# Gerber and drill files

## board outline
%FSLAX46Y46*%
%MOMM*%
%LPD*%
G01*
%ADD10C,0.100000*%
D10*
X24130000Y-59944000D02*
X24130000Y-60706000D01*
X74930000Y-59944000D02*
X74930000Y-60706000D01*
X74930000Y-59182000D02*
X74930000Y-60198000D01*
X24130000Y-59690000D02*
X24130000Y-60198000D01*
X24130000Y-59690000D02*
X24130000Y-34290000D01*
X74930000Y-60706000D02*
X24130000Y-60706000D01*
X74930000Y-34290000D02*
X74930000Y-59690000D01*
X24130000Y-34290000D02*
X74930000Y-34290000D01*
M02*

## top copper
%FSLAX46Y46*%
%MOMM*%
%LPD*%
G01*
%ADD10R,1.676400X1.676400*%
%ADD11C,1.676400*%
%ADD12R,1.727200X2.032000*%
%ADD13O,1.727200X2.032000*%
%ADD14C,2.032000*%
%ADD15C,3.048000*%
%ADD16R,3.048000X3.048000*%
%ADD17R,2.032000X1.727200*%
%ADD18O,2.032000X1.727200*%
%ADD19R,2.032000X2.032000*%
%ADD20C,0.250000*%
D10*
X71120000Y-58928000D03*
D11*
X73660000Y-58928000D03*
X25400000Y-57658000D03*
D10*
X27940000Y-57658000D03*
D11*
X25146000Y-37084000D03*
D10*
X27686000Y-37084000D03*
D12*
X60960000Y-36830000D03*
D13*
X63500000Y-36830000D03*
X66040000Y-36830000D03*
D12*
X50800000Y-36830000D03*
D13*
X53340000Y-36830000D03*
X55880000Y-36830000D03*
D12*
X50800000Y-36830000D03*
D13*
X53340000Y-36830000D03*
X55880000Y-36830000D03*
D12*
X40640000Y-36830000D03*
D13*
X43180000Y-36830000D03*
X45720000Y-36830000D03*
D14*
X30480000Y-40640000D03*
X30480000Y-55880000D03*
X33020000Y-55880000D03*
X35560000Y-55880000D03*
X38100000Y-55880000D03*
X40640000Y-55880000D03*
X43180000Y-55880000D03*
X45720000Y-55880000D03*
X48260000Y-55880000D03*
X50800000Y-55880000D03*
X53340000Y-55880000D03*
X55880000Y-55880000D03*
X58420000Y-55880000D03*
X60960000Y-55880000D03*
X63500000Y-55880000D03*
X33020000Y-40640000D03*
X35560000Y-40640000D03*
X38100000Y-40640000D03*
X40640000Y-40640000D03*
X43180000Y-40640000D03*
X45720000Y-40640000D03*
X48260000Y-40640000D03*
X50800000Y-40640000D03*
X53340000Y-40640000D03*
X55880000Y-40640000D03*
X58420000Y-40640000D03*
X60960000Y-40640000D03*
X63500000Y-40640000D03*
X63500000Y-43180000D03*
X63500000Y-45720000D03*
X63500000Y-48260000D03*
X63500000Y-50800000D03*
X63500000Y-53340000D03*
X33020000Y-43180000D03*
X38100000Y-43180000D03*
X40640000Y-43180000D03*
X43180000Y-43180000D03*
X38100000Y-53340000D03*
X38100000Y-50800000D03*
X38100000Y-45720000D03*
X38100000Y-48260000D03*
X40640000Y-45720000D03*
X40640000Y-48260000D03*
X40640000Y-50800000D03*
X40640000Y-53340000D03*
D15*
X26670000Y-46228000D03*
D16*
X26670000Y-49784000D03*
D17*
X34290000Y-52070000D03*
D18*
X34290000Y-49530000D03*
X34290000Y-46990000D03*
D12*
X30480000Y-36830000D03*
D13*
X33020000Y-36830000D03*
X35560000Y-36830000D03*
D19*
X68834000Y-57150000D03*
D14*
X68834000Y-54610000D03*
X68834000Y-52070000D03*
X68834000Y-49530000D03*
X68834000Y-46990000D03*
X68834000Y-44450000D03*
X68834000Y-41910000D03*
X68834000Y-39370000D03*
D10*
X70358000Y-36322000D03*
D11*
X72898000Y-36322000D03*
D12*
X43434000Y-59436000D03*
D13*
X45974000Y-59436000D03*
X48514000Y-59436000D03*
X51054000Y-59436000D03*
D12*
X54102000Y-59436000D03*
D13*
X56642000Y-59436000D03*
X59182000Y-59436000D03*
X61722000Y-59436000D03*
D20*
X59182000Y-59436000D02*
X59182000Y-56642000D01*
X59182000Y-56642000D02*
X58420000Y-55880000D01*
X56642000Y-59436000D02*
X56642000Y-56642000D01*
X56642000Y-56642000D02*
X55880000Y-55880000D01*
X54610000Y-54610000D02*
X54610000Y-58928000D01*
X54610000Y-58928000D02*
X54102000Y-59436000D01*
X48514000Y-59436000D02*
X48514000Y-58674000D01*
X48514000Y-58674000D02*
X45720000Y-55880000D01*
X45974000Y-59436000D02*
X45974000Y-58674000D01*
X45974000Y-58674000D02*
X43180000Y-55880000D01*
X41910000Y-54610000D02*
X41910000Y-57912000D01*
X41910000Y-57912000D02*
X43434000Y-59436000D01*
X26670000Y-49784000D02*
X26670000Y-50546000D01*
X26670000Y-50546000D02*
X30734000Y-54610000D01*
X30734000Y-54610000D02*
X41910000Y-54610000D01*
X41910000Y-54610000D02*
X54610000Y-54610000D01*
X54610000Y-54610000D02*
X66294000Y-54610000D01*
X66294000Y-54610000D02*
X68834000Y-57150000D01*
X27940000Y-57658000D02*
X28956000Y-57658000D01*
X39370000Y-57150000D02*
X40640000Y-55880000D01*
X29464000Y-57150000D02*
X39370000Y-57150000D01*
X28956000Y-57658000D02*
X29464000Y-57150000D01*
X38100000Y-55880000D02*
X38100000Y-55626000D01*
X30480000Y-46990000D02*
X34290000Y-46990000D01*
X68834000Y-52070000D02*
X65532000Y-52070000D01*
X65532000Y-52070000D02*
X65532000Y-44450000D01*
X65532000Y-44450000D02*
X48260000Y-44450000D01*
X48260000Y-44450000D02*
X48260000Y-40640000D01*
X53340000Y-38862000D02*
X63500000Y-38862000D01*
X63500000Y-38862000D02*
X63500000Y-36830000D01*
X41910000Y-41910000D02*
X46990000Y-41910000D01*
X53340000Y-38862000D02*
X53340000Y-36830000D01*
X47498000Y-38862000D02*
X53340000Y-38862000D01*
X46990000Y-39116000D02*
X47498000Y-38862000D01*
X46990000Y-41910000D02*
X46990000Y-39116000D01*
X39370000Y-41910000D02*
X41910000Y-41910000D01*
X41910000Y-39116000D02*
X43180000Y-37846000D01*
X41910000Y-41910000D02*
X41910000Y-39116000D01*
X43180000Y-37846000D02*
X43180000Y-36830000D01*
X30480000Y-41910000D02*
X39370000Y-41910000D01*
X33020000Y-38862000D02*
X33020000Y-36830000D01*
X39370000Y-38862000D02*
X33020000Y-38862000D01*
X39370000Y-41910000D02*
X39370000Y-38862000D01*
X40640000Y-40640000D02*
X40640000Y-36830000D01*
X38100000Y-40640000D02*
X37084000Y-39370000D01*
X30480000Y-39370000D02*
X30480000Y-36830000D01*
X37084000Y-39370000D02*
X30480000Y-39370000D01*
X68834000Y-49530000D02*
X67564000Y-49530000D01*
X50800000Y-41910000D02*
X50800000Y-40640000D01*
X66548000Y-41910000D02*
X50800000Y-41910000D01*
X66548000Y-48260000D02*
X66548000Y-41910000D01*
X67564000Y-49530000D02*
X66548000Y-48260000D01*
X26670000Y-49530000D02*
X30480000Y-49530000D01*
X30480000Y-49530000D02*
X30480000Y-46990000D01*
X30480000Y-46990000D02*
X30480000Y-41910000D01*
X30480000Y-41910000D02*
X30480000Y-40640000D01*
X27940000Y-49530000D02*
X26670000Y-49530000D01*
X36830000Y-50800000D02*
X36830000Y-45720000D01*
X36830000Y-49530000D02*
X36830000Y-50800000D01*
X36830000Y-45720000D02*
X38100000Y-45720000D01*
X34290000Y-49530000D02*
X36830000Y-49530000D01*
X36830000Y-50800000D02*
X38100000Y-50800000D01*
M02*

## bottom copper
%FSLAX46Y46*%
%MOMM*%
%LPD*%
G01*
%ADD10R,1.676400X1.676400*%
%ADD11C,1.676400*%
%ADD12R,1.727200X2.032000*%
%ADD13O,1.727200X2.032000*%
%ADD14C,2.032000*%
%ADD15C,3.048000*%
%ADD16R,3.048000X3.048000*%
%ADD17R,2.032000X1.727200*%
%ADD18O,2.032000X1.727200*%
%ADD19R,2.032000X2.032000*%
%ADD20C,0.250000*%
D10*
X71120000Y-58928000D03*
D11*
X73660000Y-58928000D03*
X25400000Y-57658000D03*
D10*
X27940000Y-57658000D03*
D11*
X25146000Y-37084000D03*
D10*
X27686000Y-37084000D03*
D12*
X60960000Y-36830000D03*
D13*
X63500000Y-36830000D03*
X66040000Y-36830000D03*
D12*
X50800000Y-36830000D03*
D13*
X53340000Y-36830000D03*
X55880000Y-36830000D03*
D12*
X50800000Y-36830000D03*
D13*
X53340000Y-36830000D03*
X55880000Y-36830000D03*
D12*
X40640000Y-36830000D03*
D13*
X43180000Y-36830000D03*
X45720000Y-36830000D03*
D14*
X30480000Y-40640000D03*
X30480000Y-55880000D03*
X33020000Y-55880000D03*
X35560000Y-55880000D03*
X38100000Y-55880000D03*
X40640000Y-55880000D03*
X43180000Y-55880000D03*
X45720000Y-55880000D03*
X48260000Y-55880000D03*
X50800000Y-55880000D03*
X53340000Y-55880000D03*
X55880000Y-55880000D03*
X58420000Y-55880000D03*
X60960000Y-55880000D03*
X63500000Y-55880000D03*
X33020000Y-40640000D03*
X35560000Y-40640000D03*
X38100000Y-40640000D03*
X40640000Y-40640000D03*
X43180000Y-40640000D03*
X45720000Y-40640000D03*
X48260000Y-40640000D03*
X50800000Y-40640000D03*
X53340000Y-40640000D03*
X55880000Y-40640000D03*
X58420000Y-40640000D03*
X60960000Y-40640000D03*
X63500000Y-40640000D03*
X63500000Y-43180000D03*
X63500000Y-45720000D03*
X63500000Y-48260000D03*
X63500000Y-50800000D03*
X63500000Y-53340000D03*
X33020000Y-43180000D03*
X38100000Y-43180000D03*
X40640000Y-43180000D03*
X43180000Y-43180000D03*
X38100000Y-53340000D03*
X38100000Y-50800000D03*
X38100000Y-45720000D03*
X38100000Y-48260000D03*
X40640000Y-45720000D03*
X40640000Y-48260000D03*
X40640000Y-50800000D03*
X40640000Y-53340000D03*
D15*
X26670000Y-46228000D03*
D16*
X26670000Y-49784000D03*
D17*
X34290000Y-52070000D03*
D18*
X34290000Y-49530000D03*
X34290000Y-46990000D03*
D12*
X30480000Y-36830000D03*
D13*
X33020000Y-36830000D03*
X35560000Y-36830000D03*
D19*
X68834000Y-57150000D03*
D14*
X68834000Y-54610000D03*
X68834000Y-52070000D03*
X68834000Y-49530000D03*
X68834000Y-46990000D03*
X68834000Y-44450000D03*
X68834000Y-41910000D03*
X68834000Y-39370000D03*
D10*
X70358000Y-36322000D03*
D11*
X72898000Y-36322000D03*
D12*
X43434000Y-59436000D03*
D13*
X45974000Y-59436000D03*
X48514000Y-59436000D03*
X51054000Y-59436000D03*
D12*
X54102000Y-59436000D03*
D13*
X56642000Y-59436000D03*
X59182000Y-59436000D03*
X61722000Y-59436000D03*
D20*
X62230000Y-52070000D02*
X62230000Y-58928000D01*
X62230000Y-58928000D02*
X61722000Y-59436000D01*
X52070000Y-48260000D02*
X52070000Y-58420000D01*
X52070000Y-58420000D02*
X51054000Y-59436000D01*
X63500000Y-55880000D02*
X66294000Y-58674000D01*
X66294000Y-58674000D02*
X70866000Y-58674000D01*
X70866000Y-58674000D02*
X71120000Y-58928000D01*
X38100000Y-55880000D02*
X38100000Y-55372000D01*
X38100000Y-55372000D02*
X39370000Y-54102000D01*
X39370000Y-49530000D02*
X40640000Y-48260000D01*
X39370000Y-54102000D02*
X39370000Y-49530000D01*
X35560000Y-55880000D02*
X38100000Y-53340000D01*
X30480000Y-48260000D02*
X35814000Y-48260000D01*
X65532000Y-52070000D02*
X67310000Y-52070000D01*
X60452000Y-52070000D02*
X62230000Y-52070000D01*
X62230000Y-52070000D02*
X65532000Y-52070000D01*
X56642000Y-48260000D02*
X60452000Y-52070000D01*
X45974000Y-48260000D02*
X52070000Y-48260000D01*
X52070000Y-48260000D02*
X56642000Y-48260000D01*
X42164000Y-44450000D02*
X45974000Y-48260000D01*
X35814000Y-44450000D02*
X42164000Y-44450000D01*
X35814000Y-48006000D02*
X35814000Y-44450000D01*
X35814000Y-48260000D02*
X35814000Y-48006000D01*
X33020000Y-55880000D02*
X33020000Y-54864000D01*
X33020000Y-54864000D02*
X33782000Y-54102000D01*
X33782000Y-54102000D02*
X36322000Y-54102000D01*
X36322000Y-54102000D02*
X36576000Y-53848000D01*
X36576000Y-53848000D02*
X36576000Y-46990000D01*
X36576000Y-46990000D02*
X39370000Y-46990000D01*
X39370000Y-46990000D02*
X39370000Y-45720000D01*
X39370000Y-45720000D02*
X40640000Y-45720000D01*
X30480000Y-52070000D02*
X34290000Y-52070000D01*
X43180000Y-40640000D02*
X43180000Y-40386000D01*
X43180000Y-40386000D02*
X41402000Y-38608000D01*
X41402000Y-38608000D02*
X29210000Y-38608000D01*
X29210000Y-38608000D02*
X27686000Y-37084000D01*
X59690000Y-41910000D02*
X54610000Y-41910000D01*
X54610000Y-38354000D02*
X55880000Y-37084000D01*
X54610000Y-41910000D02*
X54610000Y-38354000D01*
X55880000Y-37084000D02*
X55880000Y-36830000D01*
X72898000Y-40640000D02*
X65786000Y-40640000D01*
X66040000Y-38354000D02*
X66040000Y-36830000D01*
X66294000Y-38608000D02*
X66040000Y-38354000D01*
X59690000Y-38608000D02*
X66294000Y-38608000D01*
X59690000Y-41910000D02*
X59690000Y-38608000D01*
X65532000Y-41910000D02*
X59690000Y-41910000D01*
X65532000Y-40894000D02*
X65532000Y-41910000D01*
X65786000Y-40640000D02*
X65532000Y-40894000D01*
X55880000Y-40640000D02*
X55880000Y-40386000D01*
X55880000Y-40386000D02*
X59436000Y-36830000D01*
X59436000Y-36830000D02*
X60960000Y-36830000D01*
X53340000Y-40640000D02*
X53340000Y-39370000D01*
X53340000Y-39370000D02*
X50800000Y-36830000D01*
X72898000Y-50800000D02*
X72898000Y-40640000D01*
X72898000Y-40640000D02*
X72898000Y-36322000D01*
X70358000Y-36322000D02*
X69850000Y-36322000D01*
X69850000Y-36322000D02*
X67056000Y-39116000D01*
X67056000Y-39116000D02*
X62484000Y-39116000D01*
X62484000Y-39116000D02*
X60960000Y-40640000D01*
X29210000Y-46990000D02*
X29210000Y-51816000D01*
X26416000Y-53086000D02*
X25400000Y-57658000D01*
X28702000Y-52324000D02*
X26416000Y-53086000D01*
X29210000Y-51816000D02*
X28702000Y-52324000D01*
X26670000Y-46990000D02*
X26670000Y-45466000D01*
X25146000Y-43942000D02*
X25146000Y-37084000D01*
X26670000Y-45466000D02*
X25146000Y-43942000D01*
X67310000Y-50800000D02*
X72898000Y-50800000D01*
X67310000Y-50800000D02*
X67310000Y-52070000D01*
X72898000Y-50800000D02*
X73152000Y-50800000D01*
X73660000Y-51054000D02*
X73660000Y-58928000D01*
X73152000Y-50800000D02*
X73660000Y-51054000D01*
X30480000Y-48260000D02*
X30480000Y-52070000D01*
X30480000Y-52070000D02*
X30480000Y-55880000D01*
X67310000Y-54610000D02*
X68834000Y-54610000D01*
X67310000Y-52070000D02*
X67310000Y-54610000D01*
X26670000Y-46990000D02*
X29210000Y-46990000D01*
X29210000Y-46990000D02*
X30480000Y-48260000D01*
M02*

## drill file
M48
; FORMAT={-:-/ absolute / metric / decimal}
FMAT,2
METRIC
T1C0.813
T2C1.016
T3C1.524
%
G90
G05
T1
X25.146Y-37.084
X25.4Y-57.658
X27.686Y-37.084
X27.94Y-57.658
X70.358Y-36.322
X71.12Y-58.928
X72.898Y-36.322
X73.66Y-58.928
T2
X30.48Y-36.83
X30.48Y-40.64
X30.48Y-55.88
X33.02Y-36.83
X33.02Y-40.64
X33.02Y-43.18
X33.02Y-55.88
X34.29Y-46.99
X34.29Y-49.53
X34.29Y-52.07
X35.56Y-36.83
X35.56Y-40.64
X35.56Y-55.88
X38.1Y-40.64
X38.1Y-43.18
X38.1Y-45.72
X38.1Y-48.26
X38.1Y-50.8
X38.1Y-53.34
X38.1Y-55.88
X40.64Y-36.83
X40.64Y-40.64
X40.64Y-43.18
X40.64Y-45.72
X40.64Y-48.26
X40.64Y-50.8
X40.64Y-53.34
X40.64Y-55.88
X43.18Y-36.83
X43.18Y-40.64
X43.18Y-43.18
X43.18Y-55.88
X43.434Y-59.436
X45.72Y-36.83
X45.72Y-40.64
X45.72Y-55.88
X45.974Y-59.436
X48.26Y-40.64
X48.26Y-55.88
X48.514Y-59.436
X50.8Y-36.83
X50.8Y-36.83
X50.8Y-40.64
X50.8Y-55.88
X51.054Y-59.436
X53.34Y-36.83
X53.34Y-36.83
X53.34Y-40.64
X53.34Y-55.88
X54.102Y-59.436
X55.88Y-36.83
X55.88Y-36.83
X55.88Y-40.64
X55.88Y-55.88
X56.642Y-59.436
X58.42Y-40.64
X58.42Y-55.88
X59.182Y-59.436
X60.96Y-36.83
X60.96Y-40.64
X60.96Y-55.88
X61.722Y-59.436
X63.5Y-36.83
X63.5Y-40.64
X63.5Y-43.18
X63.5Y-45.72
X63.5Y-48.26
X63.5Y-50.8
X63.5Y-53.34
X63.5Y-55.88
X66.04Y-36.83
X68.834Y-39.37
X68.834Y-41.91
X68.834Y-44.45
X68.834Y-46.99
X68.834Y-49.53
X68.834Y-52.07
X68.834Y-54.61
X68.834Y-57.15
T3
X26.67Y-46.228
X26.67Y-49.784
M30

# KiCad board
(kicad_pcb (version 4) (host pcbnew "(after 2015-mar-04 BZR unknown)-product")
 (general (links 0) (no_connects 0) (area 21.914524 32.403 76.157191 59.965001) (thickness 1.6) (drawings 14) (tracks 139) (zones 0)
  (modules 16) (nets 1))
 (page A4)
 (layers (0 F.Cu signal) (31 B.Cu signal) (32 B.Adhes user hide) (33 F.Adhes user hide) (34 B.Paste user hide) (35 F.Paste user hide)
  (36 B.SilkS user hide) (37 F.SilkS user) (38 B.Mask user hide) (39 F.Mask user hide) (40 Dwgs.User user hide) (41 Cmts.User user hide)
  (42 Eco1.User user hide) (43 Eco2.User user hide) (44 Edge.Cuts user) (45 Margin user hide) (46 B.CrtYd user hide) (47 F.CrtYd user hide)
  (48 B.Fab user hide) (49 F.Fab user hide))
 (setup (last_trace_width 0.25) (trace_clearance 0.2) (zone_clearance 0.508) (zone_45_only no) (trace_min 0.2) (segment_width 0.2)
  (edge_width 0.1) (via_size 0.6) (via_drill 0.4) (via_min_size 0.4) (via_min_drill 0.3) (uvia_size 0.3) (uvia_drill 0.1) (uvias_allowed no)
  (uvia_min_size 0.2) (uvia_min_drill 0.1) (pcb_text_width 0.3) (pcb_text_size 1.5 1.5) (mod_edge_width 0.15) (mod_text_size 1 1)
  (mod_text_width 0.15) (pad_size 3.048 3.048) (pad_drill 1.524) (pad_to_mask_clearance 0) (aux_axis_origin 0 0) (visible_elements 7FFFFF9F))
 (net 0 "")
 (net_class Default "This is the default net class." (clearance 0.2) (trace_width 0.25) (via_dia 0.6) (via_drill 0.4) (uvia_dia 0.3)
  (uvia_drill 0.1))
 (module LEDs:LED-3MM (layer F.Cu) (at 72.39 58.928)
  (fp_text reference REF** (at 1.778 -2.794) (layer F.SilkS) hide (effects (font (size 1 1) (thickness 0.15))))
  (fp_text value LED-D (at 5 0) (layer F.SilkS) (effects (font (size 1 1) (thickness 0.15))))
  (pad 1 thru_hole rect (at -1.27 0) (size 1.6764 1.6764) (drill 0.8128) (layers *.Cu *.Mask F.SilkS))
  (pad 2 thru_hole circle (at 1.27 0) (size 1.6764 1.6764) (drill 0.8128) (layers *.Cu *.Mask F.SilkS)))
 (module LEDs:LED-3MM (layer F.Cu) (at 26.67 57.658)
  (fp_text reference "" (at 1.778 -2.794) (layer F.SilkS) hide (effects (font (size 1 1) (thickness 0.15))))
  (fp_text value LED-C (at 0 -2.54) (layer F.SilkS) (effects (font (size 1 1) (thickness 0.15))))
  (pad 1 thru_hole circle (at -1.27 0) (size 1.6764 1.6764) (drill 0.8128) (layers *.Cu *.Mask F.SilkS))
  (pad 2 thru_hole rect (at 1.27 0) (size 1.6764 1.6764) (drill 0.8128) (layers *.Cu *.Mask F.SilkS)))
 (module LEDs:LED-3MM (layer F.Cu) (at 26.416 37.084)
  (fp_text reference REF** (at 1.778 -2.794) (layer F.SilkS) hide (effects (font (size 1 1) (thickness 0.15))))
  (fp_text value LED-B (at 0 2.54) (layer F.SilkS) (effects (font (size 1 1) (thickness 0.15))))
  (pad 1 thru_hole circle (at -1.27 0) (size 1.6764 1.6764) (drill 0.8128) (layers *.Cu *.Mask F.SilkS))
  (pad 2 thru_hole rect (at 1.27 0) (size 1.6764 1.6764) (drill 0.8128) (layers *.Cu *.Mask F.SilkS)))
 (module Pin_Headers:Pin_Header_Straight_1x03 (layer F.Cu) (at 60.96 36.83 90)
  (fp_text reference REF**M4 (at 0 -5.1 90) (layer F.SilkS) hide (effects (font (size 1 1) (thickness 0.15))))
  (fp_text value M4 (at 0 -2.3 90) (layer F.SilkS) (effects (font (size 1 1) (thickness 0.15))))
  (pad 1 thru_hole rect (at 0 0 90) (size 2.032 1.7272) (drill 1.016) (layers *.Cu *.Mask F.SilkS))
  (pad 2 thru_hole oval (at 0 2.54 90) (size 2.032 1.7272) (drill 1.016) (layers *.Cu *.Mask F.SilkS))
  (pad 3 thru_hole oval (at 0 5.08 90) (size 2.032 1.7272) (drill 1.016) (layers *.Cu *.Mask F.SilkS)))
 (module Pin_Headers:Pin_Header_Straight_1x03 (layer F.Cu) (at 50.8 36.83 90)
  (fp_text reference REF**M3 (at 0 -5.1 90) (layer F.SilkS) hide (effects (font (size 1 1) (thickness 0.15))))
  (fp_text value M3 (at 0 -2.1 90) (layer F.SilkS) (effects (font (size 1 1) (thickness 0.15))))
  (pad 1 thru_hole rect (at 0 0 90) (size 2.032 1.7272) (drill 1.016) (layers *.Cu *.Mask F.SilkS))
  (pad 2 thru_hole oval (at 0 2.54 90) (size 2.032 1.7272) (drill 1.016) (layers *.Cu *.Mask F.SilkS))
  (pad 3 thru_hole oval (at 0 5.08 90) (size 2.032 1.7272) (drill 1.016) (layers *.Cu *.Mask F.SilkS)))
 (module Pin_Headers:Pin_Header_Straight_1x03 (layer F.Cu) (at 50.8 36.83 90)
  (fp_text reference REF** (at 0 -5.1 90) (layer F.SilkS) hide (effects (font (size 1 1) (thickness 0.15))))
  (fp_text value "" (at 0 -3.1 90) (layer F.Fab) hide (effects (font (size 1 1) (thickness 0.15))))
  (pad 1 thru_hole rect (at 0 0 90) (size 2.032 1.7272) (drill 1.016) (layers *.Cu *.Mask F.SilkS))
  (pad 2 thru_hole oval (at 0 2.54 90) (size 2.032 1.7272) (drill 1.016) (layers *.Cu *.Mask F.SilkS))
  (pad 3 thru_hole oval (at 0 5.08 90) (size 2.032 1.7272) (drill 1.016) (layers *.Cu *.Mask F.SilkS)))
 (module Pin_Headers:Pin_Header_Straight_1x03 (layer F.Cu) (at 40.64 36.83 90)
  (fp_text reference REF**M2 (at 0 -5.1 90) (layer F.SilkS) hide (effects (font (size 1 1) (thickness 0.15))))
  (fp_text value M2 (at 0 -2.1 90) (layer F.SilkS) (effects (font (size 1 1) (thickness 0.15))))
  (pad 1 thru_hole rect (at 0 0 90) (size 2.032 1.7272) (drill 1.016) (layers *.Cu *.Mask F.SilkS))
  (pad 2 thru_hole oval (at 0 2.54 90) (size 2.032 1.7272) (drill 1.016) (layers *.Cu *.Mask F.SilkS))
  (pad 3 thru_hole oval (at 0 5.08 90) (size 2.032 1.7272) (drill 1.016) (layers *.Cu *.Mask F.SilkS)))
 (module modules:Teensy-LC (layer F.Cu) (at 45.72 48.26)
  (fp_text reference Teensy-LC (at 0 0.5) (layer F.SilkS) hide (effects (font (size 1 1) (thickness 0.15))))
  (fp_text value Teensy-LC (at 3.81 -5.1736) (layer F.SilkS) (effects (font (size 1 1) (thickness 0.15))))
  (pad 5v thru_hole circle (at -15.24 -7.62) (size 2.032 2.032) (drill 1.016) (layers *.Cu *.Mask F.SilkS))
  (pad GND thru_hole circle (at -15.24 7.62) (size 2.032 2.032) (drill 1.016) (layers *.Cu *.Mask F.SilkS))
  (pad 0 thru_hole circle (at -12.7 7.62) (size 2.032 2.032) (drill 1.016) (layers *.Cu *.Mask F.SilkS))
  (pad 1 thru_hole circle (at -10.16 7.62) (size 2.032 2.032) (drill 1.016) (layers *.Cu *.Mask F.SilkS))
  (pad 2 thru_hole circle (at -7.62 7.62) (size 2.032 2.032) (drill 1.016) (layers *.Cu *.Mask F.SilkS))
  (pad 3 thru_hole circle (at -5.08 7.62) (size 2.032 2.032) (drill 1.016) (layers *.Cu *.Mask F.SilkS))
  (pad 4 thru_hole circle (at -2.54 7.62) (size 2.032 2.032) (drill 1.016) (layers *.Cu *.Mask F.SilkS))
  (pad 5 thru_hole circle (at 0 7.62) (size 2.032 2.032) (drill 1.016) (layers *.Cu *.Mask F.SilkS))
  (pad 6 thru_hole circle (at 2.54 7.62) (size 2.032 2.032) (drill 1.016) (layers *.Cu *.Mask F.SilkS))
  (pad 7 thru_hole circle (at 5.08 7.62) (size 2.032 2.032) (drill 1.016) (layers *.Cu *.Mask F.SilkS))
  (pad 8 thru_hole circle (at 7.62 7.62) (size 2.032 2.032) (drill 1.016) (layers *.Cu *.Mask F.SilkS))
  (pad 9 thru_hole circle (at 10.16 7.62) (size 2.032 2.032) (drill 1.016) (layers *.Cu *.Mask F.SilkS))
  (pad 10 thru_hole circle (at 12.7 7.62) (size 2.032 2.032) (drill 1.016) (layers *.Cu *.Mask F.SilkS))
  (pad 11 thru_hole circle (at 15.24 7.62) (size 2.032 2.032) (drill 1.016) (layers *.Cu *.Mask F.SilkS))
  (pad 12 thru_hole circle (at 17.78 7.62) (size 2.032 2.032) (drill 1.016) (layers *.Cu *.Mask F.SilkS))
  (pad GND thru_hole circle (at -12.7 -7.62) (size 2.032 2.032) (drill 1.016) (layers *.Cu *.Mask F.SilkS))
  (pad 3.3v thru_hole circle (at -10.16 -7.62) (size 2.032 2.032) (drill 1.016) (layers *.Cu *.Mask F.SilkS))
  (pad 23 thru_hole circle (at -7.62 -7.62) (size 2.032 2.032) (drill 1.016) (layers *.Cu *.Mask F.SilkS))
  (pad 22 thru_hole circle (at -5.08 -7.62) (size 2.032 2.032) (drill 1.016) (layers *.Cu *.Mask F.SilkS))
  (pad 21 thru_hole circle (at -2.54 -7.62) (size 2.032 2.032) (drill 1.016) (layers *.Cu *.Mask F.SilkS))
  (pad 20 thru_hole circle (at 0 -7.62) (size 2.032 2.032) (drill 1.016) (layers *.Cu *.Mask F.SilkS))
  (pad 19 thru_hole circle (at 2.54 -7.62) (size 2.032 2.032) (drill 1.016) (layers *.Cu *.Mask F.SilkS))
  (pad 18 thru_hole circle (at 5.08 -7.62) (size 2.032 2.032) (drill 1.016) (layers *.Cu *.Mask F.SilkS))
  (pad 17 thru_hole circle (at 7.62 -7.62) (size 2.032 2.032) (drill 1.016) (layers *.Cu *.Mask F.SilkS))
  (pad 16 thru_hole circle (at 10.16 -7.62) (size 2.032 2.032) (drill 1.016) (layers *.Cu *.Mask F.SilkS))
  (pad 15 thru_hole circle (at 12.7 -7.62) (size 2.032 2.032) (drill 1.016) (layers *.Cu *.Mask F.SilkS))
  (pad 14 thru_hole circle (at 15.24 -7.62) (size 2.032 2.032) (drill 1.016) (layers *.Cu *.Mask F.SilkS))
  (pad 13 thru_hole circle (at 17.78 -7.62) (size 2.032 2.032) (drill 1.016) (layers *.Cu *.Mask F.SilkS))
  (pad DAC thru_hole circle (at 17.78 -5.08) (size 2.032 2.032) (drill 1.016) (layers *.Cu *.Mask F.SilkS))
  (pad PGR thru_hole circle (at 17.78 -2.54) (size 2.032 2.032) (drill 1.016) (layers *.Cu *.Mask F.SilkS))
  (pad GND thru_hole circle (at 17.78 0) (size 2.032 2.032) (drill 1.016) (layers *.Cu *.Mask F.SilkS))
  (pad 3.3v thru_hole circle (at 17.78 2.54) (size 2.032 2.032) (drill 1.016) (layers *.Cu *.Mask F.SilkS))
  (pad 17 thru_hole circle (at 17.78 5.08) (size 2.032 2.032) (drill 1.016) (layers *.Cu *.Mask F.SilkS))
  (pad VUSB thru_hole circle (at -12.7 -5.08) (size 2.032 2.032) (drill 1.016) (layers *.Cu *.Mask F.SilkS))
  (pad AREF thru_hole circle (at -7.62 -5.08) (size 2.032 2.032) (drill 1.016) (layers *.Cu *.Mask F.SilkS))
  (pad 24 thru_hole circle (at -5.08 -5.08) (size 2.032 2.032) (drill 1.016) (layers *.Cu *.Mask F.SilkS))
  (pad 25 thru_hole circle (at -2.54 -5.08) (size 2.032 2.032) (drill 1.016) (layers *.Cu *.Mask F.SilkS)))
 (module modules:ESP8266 (layer B.Cu) (at 50.8 48.26)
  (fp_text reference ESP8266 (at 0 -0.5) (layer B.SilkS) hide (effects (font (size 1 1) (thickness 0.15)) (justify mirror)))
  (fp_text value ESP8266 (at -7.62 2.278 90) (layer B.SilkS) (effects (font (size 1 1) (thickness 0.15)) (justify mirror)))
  (pad TX thru_hole circle (at -12.7 5.08) (size 2.032 2.032) (drill 1.016) (layers *.Cu *.Mask B.SilkS))
  (pad CH thru_hole circle (at -12.7 2.54) (size 2.032 2.032) (drill 1.016) (layers *.Cu *.Mask B.SilkS))
  (pad VCC thru_hole circle (at -12.7 -2.54) (size 2.032 2.032) (drill 1.016) (layers *.Cu *.Mask B.SilkS))
  (pad RST thru_hole circle (at -12.7 0) (size 2.032 2.032) (drill 1.016) (layers *.Cu *.Mask B.SilkS))
  (pad RX thru_hole circle (at -10.16 -2.54) (size 2.032 2.032) (drill 1.016) (layers *.Cu *.Mask B.SilkS))
  (pad G0 thru_hole circle (at -10.16 0) (size 2.032 2.032) (drill 1.016) (layers *.Cu *.Mask B.SilkS))
  (pad G1 thru_hole circle (at -10.16 2.54) (size 2.032 2.032) (drill 1.016) (layers *.Cu *.Mask B.SilkS))
  (pad GND thru_hole circle (at -10.16 5.08) (size 2.032 2.032) (drill 1.016) (layers *.Cu *.Mask B.SilkS)))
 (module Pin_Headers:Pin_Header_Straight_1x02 (layer F.Cu) (at 26.67 46.99)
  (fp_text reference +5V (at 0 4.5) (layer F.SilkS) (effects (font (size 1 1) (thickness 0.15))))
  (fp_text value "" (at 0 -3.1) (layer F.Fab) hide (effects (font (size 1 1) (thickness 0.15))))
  (pad GND thru_hole circle (at 0 -0.762) (size 3.048 3.048) (drill 1.524) (layers *.Cu *.Mask F.SilkS))
  (pad 5V thru_hole rect (at 0 2.794) (size 3.048 3.048) (drill 1.524) (layers *.Cu *.Mask F.SilkS)))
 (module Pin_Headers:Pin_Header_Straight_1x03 (layer F.Cu) (at 34.29 52.07 180)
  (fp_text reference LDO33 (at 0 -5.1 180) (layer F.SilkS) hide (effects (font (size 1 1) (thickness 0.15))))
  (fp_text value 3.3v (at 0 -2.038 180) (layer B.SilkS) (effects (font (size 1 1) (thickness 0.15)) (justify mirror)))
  (pad GND thru_hole rect (at 0 0 180) (size 2.032 1.7272) (drill 1.016) (layers *.Cu *.Mask F.SilkS))
  (pad 3.3 thru_hole oval (at 0 2.54 180) (size 2.032 1.7272) (drill 1.016) (layers *.Cu *.Mask F.SilkS))
  (pad 5V thru_hole oval (at 0 5.08 180) (size 2.032 1.7272) (drill 1.016) (layers *.Cu *.Mask F.SilkS)))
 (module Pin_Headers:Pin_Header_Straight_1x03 (layer F.Cu) (at 30.48 36.83 90)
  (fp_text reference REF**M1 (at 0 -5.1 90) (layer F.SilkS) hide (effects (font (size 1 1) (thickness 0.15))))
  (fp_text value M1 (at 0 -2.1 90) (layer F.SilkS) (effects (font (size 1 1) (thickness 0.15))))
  (pad 1 thru_hole rect (at 0 0 90) (size 2.032 1.7272) (drill 1.016) (layers *.Cu *.Mask F.SilkS))
  (pad 2 thru_hole oval (at 0 2.54 90) (size 2.032 1.7272) (drill 1.016) (layers *.Cu *.Mask F.SilkS))
  (pad 3 thru_hole oval (at 0 5.08 90) (size 2.032 1.7272) (drill 1.016) (layers *.Cu *.Mask F.SilkS)))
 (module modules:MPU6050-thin (layer F.Cu) (at 73.914 49.53 90)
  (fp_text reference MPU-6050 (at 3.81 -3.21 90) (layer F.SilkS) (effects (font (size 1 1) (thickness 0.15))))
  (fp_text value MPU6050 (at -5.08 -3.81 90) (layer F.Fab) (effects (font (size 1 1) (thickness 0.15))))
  (pad VCC thru_hole rect (at -7.62 -5.08 180) (size 2.032 2.032) (drill 1.016) (layers *.Cu *.Mask F.SilkS))
  (pad GND thru_hole circle (at -5.08 -5.08 90) (size 2.032 2.032) (drill 1.016) (layers *.Cu *.Mask F.SilkS))
  (pad SCL thru_hole circle (at -2.54 -5.08 90) (size 2.032 2.032) (drill 1.016) (layers *.Cu *.Mask F.SilkS))
  (pad SDA thru_hole circle (at 0 -5.08 90) (size 2.032 2.032) (drill 1.016) (layers *.Cu *.Mask F.SilkS))
  (pad XCL thru_hole circle (at 2.54 -5.08 90) (size 2.032 2.032) (drill 1.016) (layers *.Cu *.Mask F.SilkS))
  (pad XDA thru_hole circle (at 5.08 -5.08 90) (size 2.032 2.032) (drill 1.016) (layers *.Cu *.Mask F.SilkS))
  (pad ADD thru_hole circle (at 7.62 -5.08 90) (size 2.032 2.032) (drill 1.016) (layers *.Cu *.Mask F.SilkS))
  (pad INI thru_hole circle (at 10.16 -5.08 90) (size 2.032 2.032) (drill 1.016) (layers *.Cu *.Mask F.SilkS)))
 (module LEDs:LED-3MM (layer F.Cu) (at 71.628 36.322)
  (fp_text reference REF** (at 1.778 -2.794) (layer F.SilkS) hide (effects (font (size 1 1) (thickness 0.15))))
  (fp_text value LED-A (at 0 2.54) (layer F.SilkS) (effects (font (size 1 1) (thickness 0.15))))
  (pad 1 thru_hole rect (at -1.27 0) (size 1.6764 1.6764) (drill 0.8128) (layers *.Cu *.Mask F.SilkS))
  (pad 2 thru_hole circle (at 1.27 0) (size 1.6764 1.6764) (drill 0.8128) (layers *.Cu *.Mask F.SilkS)))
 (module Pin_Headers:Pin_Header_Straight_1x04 (layer F.Cu) (at 43.434 59.436 90)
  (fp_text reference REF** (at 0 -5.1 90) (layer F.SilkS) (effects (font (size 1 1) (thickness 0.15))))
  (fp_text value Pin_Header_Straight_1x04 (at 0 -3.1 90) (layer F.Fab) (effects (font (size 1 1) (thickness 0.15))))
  (pad 1 thru_hole rect (at 0 0 90) (size 2.032 1.7272) (drill 1.016) (layers *.Cu *.Mask F.SilkS))
  (pad 2 thru_hole oval (at 0 2.54 90) (size 2.032 1.7272) (drill 1.016) (layers *.Cu *.Mask F.SilkS))
  (pad 3 thru_hole oval (at 0 5.08 90) (size 2.032 1.7272) (drill 1.016) (layers *.Cu *.Mask F.SilkS))
  (pad 4 thru_hole oval (at 0 7.62 90) (size 2.032 1.7272) (drill 1.016) (layers *.Cu *.Mask F.SilkS)))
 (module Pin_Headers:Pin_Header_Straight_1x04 (layer F.Cu) (at 54.102 59.436 90)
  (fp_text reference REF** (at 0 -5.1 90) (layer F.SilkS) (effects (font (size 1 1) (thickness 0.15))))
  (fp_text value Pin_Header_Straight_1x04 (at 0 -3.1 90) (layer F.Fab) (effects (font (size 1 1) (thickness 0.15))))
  (pad 1 thru_hole rect (at 0 0 90) (size 2.032 1.7272) (drill 1.016) (layers *.Cu *.Mask F.SilkS))
  (pad 2 thru_hole oval (at 0 2.54 90) (size 2.032 1.7272) (drill 1.016) (layers *.Cu *.Mask F.SilkS))
  (pad 3 thru_hole oval (at 0 5.08 90) (size 2.032 1.7272) (drill 1.016) (layers *.Cu *.Mask F.SilkS))
  (pad 4 thru_hole oval (at 0 7.62 90) (size 2.032 1.7272) (drill 1.016) (layers *.Cu *.Mask F.SilkS)))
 (gr_line (start 24.13 59.944) (end 24.13 60.706) (angle 90) (layer Edge.Cuts) (width 0.1))
 (gr_line (start 74.93 59.944) (end 74.93 60.706) (angle 90) (layer Edge.Cuts) (width 0.1))
 (gr_line (start 74.93 59.182) (end 74.93 60.198) (angle 90) (layer Edge.Cuts) (width 0.1))
 (gr_line (start 24.13 59.69) (end 24.13 60.198) (angle 90) (layer Edge.Cuts) (width 0.1))
 (gr_line (start 24.13 59.69) (end 24.13 34.29) (angle 90) (layer Edge.Cuts) (width 0.1))
 (gr_line (start 74.93 60.706) (end 24.13 60.706) (angle 90) (layer Edge.Cuts) (width 0.1))
 (gr_line (start 74.93 34.29) (end 74.93 59.69) (angle 90) (layer Edge.Cuts) (width 0.1))
 (gr_line (start 24.13 34.29) (end 74.93 34.29) (angle 90) (layer Edge.Cuts) (width 0.1))
 (segment (start 59.182 59.436) (end 59.182 56.642) (width 0.25) (layer F.Cu) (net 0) (status 400000))
 (segment (start 59.182 56.642) (end 58.42 55.88) (width 0.25) (layer F.Cu) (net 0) (status 800000))
 (segment (start 56.642 59.436) (end 56.642 56.642) (width 0.25) (layer F.Cu) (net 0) (status 400000))
 (segment (start 56.642 56.642) (end 55.88 55.88) (width 0.25) (layer F.Cu) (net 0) (status 800000))
 (segment (start 62.23 52.07) (end 62.23 58.928) (width 0.25) (layer B.Cu) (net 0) (status 800000))
 (segment (start 62.23 58.928) (end 61.722 59.436) (width 0.25) (layer B.Cu) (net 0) (status C00000))
 (segment (start 54.61 54.61) (end 54.61 58.928) (width 0.25) (layer F.Cu) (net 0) (status 800000))
 (segment (start 54.61 58.928) (end 54.102 59.436) (width 0.25) (layer F.Cu) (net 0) (status C00000))
 (segment (start 48.514 59.436) (end 48.514 58.674) (width 0.25) (layer F.Cu) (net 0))
 (segment (start 48.514 58.674) (end 45.72 55.88) (width 0.25) (layer F.Cu) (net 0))
 (segment (start 45.974 59.436) (end 45.974 58.674) (width 0.25) (layer F.Cu) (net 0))
 (segment (start 45.974 58.674) (end 43.18 55.88) (width 0.25) (layer F.Cu) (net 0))
 (segment (start 52.07 48.26) (end 52.07 58.42) (width 0.25) (layer B.Cu) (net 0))
 (segment (start 52.07 58.42) (end 51.054 59.436) (width 0.25) (layer B.Cu) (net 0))
 (segment (start 41.91 54.61) (end 41.91 57.912) (width 0.25) (layer F.Cu) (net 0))
 (segment (start 41.91 57.912) (end 43.434 59.436) (width 0.25) (layer F.Cu) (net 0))
 (segment (start 63.5 55.88) (end 66.294 58.674) (width 0.25) (layer B.Cu) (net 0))
 (segment (start 66.294 58.674) (end 70.866 58.674) (width 0.25) (layer B.Cu) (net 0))
 (segment (start 70.866 58.674) (end 71.12 58.928) (width 0.25) (layer B.Cu) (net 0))
 (segment (start 38.1 55.88) (end 38.1 55.372) (width 0.25) (layer B.Cu) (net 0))
 (segment (start 38.1 55.372) (end 39.37 54.102) (width 0.25) (layer B.Cu) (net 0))
 (segment (start 39.37 49.53) (end 40.64 48.26) (width 0.25) (layer B.Cu) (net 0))
 (segment (start 39.37 54.102) (end 39.37 49.53) (width 0.25) (layer B.Cu) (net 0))
 (segment (start 35.56 55.88) (end 38.1 53.34) (width 0.25) (layer B.Cu) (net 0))
 (segment (start 26.67 49.784) (end 26.67 50.546) (width 0.25) (layer F.Cu) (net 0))
 (segment (start 26.67 50.546) (end 30.734 54.61) (width 0.25) (layer F.Cu) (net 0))
 (segment (start 30.734 54.61) (end 41.91 54.61) (width 0.25) (layer F.Cu) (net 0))
 (segment (start 41.91 54.61) (end 54.61 54.61) (width 0.25) (layer F.Cu) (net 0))
 (segment (start 54.61 54.61) (end 66.294 54.61) (width 0.25) (layer F.Cu) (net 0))
 (segment (start 66.294 54.61) (end 68.834 57.15) (width 0.25) (layer F.Cu) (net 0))
 (segment (start 27.94 57.658) (end 28.956 57.658) (width 0.25) (layer F.Cu) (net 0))
 (segment (start 39.37 57.15) (end 40.64 55.88) (width 0.25) (layer F.Cu) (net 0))
 (segment (start 29.464 57.15) (end 39.37 57.15) (width 0.25) (layer F.Cu) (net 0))
 (segment (start 28.956 57.658) (end 29.464 57.15) (width 0.25) (layer F.Cu) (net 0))
 (segment (start 30.48 48.26) (end 35.814 48.26) (width 0.25) (layer B.Cu) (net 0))
 (segment (start 65.532 52.07) (end 67.31 52.07) (width 0.25) (layer B.Cu) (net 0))
 (segment (start 60.452 52.07) (end 62.23 52.07) (width 0.25) (layer B.Cu) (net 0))
 (segment (start 62.23 52.07) (end 65.532 52.07) (width 0.25) (layer B.Cu) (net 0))
 (segment (start 56.642 48.26) (end 60.452 52.07) (width 0.25) (layer B.Cu) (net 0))
 (segment (start 45.974 48.26) (end 52.07 48.26) (width 0.25) (layer B.Cu) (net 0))
 (segment (start 52.07 48.26) (end 56.642 48.26) (width 0.25) (layer B.Cu) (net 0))
 (segment (start 42.164 44.45) (end 45.974 48.26) (width 0.25) (layer B.Cu) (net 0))
 (segment (start 35.814 44.45) (end 42.164 44.45) (width 0.25) (layer B.Cu) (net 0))
 (segment (start 35.814 48.006) (end 35.814 44.45) (width 0.25) (layer B.Cu) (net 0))
 (segment (start 35.814 48.26) (end 35.814 48.006) (width 0.25) (layer B.Cu) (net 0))
 (segment (start 38.1 55.88) (end 38.1 55.626) (width 0.25) (layer F.Cu) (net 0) (status 30))
 (segment (start 33.02 55.88) (end 33.02 54.864) (width 0.25) (layer B.Cu) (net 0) (status 30))
 (segment (start 33.02 54.864) (end 33.782 54.102) (width 0.25) (layer B.Cu) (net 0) (status 10))
 (segment (start 33.782 54.102) (end 36.322 54.102) (width 0.25) (layer B.Cu) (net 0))
 (segment (start 36.322 54.102) (end 36.576 53.848) (width 0.25) (layer B.Cu) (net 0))
 (segment (start 36.576 53.848) (end 36.576 46.99) (width 0.25) (layer B.Cu) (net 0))
 (segment (start 36.576 46.99) (end 39.37 46.99) (width 0.25) (layer B.Cu) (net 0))
 (segment (start 39.37 46.99) (end 39.37 45.72) (width 0.25) (layer B.Cu) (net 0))
 (segment (start 39.37 45.72) (end 40.64 45.72) (width 0.25) (layer B.Cu) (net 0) (status 20))
 (segment (start 30.48 46.99) (end 34.29 46.99) (width 0.25) (layer F.Cu) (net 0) (status 20))
 (segment (start 30.48 52.07) (end 34.29 52.07) (width 0.25) (layer B.Cu) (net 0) (status 20))
 (segment (start 68.834 52.07) (end 65.532 52.07) (width 0.25) (layer F.Cu) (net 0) (status 10))
 (segment (start 65.532 52.07) (end 65.532 44.45) (width 0.25) (layer F.Cu) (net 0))
 (segment (start 65.532 44.45) (end 48.26 44.45) (width 0.25) (layer F.Cu) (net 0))
 (segment (start 48.26 44.45) (end 48.26 40.64) (width 0.25) (layer F.Cu) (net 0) (status 20))
 (segment (start 43.18 40.64) (end 43.18 40.386) (width 0.25) (layer B.Cu) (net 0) (status 30))
 (segment (start 43.18 40.386) (end 41.402 38.608) (width 0.25) (layer B.Cu) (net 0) (status 10))
 (segment (start 41.402 38.608) (end 29.21 38.608) (width 0.25) (layer B.Cu) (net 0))
 (segment (start 29.21 38.608) (end 27.686 37.084) (width 0.25) (layer B.Cu) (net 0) (status 20))
 (segment (start 59.69 41.91) (end 54.61 41.91) (width 0.25) (layer B.Cu) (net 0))
 (segment (start 54.61 38.354) (end 55.88 37.084) (width 0.25) (layer B.Cu) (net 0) (status 20))
 (segment (start 54.61 41.91) (end 54.61 38.354) (width 0.25) (layer B.Cu) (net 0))
 (segment (start 55.88 37.084) (end 55.88 36.83) (width 0.25) (layer B.Cu) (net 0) (status 30))
 (segment (start 72.898 40.64) (end 65.786 40.64) (width 0.25) (layer B.Cu) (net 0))
 (segment (start 66.04 38.354) (end 66.04 36.83) (width 0.25) (layer B.Cu) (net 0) (status 20))
 (segment (start 66.294 38.608) (end 66.04 38.354) (width 0.25) (layer B.Cu) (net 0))
 (segment (start 59.69 38.608) (end 66.294 38.608) (width 0.25) (layer B.Cu) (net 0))
 (segment (start 59.69 41.91) (end 59.69 38.608) (width 0.25) (layer B.Cu) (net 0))
 (segment (start 65.532 41.91) (end 59.69 41.91) (width 0.25) (layer B.Cu) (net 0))
 (segment (start 65.532 40.894) (end 65.532 41.91) (width 0.25) (layer B.Cu) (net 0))
 (segment (start 65.786 40.64) (end 65.532 40.894) (width 0.25) (layer B.Cu) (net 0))
 (segment (start 53.34 38.862) (end 63.5 38.862) (width 0.25) (layer F.Cu) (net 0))
 (segment (start 63.5 38.862) (end 63.5 36.83) (width 0.25) (layer F.Cu) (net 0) (status 20))
 (segment (start 41.91 41.91) (end 46.99 41.91) (width 0.25) (layer F.Cu) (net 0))
 (segment (start 53.34 38.862) (end 53.34 36.83) (width 0.25) (layer F.Cu) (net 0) (status 20))
 (segment (start 47.498 38.862) (end 53.34 38.862) (width 0.25) (layer F.Cu) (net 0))
 (segment (start 46.99 39.116) (end 47.498 38.862) (width 0.25) (layer F.Cu) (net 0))
 (segment (start 46.99 41.91) (end 46.99 39.116) (width 0.25) (layer F.Cu) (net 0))
 (segment (start 55.88 40.64) (end 55.88 40.386) (width 0.25) (layer B.Cu) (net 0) (status 30))
 (segment (start 55.88 40.386) (end 59.436 36.83) (width 0.25) (layer B.Cu) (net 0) (status 10))
 (segment (start 59.436 36.83) (end 60.96 36.83) (width 0.25) (layer B.Cu) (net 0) (status 20))
 (segment (start 53.34 40.64) (end 53.34 39.37) (width 0.25) (layer B.Cu) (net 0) (status 10))
 (segment (start 53.34 39.37) (end 50.8 36.83) (width 0.25) (layer B.Cu) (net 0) (status 20))
 (segment (start 39.37 41.91) (end 41.91 41.91) (width 0.25) (layer F.Cu) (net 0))
 (segment (start 41.91 39.116) (end 43.18 37.846) (width 0.25) (layer F.Cu) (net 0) (status 20))
 (segment (start 41.91 41.91) (end 41.91 39.116) (width 0.25) (layer F.Cu) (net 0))
 (segment (start 43.18 37.846) (end 43.18 36.83) (width 0.25) (layer F.Cu) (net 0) (status 30))
 (segment (start 30.48 41.91) (end 39.37 41.91) (width 0.25) (layer F.Cu) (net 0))
 (segment (start 33.02 38.862) (end 33.02 36.83) (width 0.25) (layer F.Cu) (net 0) (status 20))
 (segment (start 39.37 38.862) (end 33.02 38.862) (width 0.25) (layer F.Cu) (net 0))
 (segment (start 39.37 41.91) (end 39.37 38.862) (width 0.25) (layer F.Cu) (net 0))
 (segment (start 40.64 40.64) (end 40.64 36.83) (width 0.25) (layer F.Cu) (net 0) (status 30))
 (segment (start 38.1 40.64) (end 37.084 39.37) (width 0.25) (layer F.Cu) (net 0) (status 10))
 (segment (start 30.48 39.37) (end 30.48 36.83) (width 0.25) (layer F.Cu) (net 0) (status 20))
 (segment (start 37.084 39.37) (end 30.48 39.37) (width 0.25) (layer F.Cu) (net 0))
 (segment (start 68.834 49.53) (end 67.564 49.53) (width 0.25) (layer F.Cu) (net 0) (status 10))
 (segment (start 50.8 41.91) (end 50.8 40.64) (width 0.25) (layer F.Cu) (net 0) (status 20))
 (segment (start 66.548 41.91) (end 50.8 41.91) (width 0.25) (layer F.Cu) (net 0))
 (segment (start 66.548 48.26) (end 66.548 41.91) (width 0.25) (layer F.Cu) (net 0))
 (segment (start 67.564 49.53) (end 66.548 48.26) (width 0.25) (layer F.Cu) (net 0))
 (segment (start 72.898 50.8) (end 72.898 40.64) (width 0.25) (layer B.Cu) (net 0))
 (segment (start 72.898 40.64) (end 72.898 36.322) (width 0.25) (layer B.Cu) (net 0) (status 20))
 (segment (start 70.358 36.322) (end 69.85 36.322) (width 0.25) (layer B.Cu) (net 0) (status 30))
 (segment (start 69.85 36.322) (end 67.056 39.116) (width 0.25) (layer B.Cu) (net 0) (status 10))
 (segment (start 67.056 39.116) (end 62.484 39.116) (width 0.25) (layer B.Cu) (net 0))
 (segment (start 62.484 39.116) (end 60.96 40.64) (width 0.25) (layer B.Cu) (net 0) (status 20))
 (segment (start 29.21 46.99) (end 29.21 51.816) (width 0.25) (layer B.Cu) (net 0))
 (segment (start 26.416 53.086) (end 25.4 57.658) (width 0.25) (layer B.Cu) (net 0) (status 20))
 (segment (start 28.702 52.324) (end 26.416 53.086) (width 0.25) (layer B.Cu) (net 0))
 (segment (start 29.21 51.816) (end 28.702 52.324) (width 0.25) (layer B.Cu) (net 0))
 (segment (start 26.67 46.99) (end 26.67 45.466) (width 0.25) (layer B.Cu) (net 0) (status 30))
 (segment (start 25.146 43.942) (end 25.146 37.084) (width 0.25) (layer B.Cu) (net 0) (status 20))
 (segment (start 26.67 45.466) (end 25.146 43.942) (width 0.25) (layer B.Cu) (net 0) (status 10))
 (segment (start 67.31 50.8) (end 72.898 50.8) (width 0.25) (layer B.Cu) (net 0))
 (segment (start 67.31 50.8) (end 67.31 52.07) (width 0.25) (layer B.Cu) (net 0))
 (segment (start 72.898 50.8) (end 73.152 50.8) (width 0.25) (layer B.Cu) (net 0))
 (segment (start 73.66 51.054) (end 73.66 58.928) (width 0.25) (layer B.Cu) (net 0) (status 20))
 (segment (start 73.152 50.8) (end 73.66 51.054) (width 0.25) (layer B.Cu) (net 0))
 (segment (start 30.48 48.26) (end 30.48 52.07) (width 0.25) (layer B.Cu) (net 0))
 (segment (start 30.48 52.07) (end 30.48 55.88) (width 0.25) (layer B.Cu) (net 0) (status 20))
 (segment (start 26.67 49.53) (end 30.48 49.53) (width 0.25) (layer F.Cu) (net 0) (status 10))
 (segment (start 30.48 49.53) (end 30.48 46.99) (width 0.25) (layer F.Cu) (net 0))
 (segment (start 30.48 46.99) (end 30.48 41.91) (width 0.25) (layer F.Cu) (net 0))
 (segment (start 30.48 41.91) (end 30.48 40.64) (width 0.25) (layer F.Cu) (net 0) (status 20))
 (segment (start 67.31 54.61) (end 68.834 54.61) (width 0.25) (layer B.Cu) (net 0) (status 20))
 (segment (start 67.31 52.07) (end 67.31 54.61) (width 0.25) (layer B.Cu) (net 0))
 (segment (start 26.67 46.99) (end 29.21 46.99) (width 0.25) (layer B.Cu) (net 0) (status 10))
 (segment (start 29.21 46.99) (end 30.48 48.26) (width 0.25) (layer B.Cu) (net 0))
 (segment (start 27.94 49.53) (end 26.67 49.53) (width 0.25) (layer F.Cu) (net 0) (status 30))
 (segment (start 36.83 50.8) (end 36.83 45.72) (width 0.25) (layer F.Cu) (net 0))
 (segment (start 36.83 49.53) (end 36.83 50.8) (width 0.25) (layer F.Cu) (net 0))
 (segment (start 36.83 45.72) (end 38.1 45.72) (width 0.25) (layer F.Cu) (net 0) (status 20))
 (segment (start 34.29 49.53) (end 36.83 49.53) (width 0.25) (layer F.Cu) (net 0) (status 10))
 (segment (start 36.83 50.8) (end 38.1 50.8) (width 0.25) (layer F.Cu) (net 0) (status 20)))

